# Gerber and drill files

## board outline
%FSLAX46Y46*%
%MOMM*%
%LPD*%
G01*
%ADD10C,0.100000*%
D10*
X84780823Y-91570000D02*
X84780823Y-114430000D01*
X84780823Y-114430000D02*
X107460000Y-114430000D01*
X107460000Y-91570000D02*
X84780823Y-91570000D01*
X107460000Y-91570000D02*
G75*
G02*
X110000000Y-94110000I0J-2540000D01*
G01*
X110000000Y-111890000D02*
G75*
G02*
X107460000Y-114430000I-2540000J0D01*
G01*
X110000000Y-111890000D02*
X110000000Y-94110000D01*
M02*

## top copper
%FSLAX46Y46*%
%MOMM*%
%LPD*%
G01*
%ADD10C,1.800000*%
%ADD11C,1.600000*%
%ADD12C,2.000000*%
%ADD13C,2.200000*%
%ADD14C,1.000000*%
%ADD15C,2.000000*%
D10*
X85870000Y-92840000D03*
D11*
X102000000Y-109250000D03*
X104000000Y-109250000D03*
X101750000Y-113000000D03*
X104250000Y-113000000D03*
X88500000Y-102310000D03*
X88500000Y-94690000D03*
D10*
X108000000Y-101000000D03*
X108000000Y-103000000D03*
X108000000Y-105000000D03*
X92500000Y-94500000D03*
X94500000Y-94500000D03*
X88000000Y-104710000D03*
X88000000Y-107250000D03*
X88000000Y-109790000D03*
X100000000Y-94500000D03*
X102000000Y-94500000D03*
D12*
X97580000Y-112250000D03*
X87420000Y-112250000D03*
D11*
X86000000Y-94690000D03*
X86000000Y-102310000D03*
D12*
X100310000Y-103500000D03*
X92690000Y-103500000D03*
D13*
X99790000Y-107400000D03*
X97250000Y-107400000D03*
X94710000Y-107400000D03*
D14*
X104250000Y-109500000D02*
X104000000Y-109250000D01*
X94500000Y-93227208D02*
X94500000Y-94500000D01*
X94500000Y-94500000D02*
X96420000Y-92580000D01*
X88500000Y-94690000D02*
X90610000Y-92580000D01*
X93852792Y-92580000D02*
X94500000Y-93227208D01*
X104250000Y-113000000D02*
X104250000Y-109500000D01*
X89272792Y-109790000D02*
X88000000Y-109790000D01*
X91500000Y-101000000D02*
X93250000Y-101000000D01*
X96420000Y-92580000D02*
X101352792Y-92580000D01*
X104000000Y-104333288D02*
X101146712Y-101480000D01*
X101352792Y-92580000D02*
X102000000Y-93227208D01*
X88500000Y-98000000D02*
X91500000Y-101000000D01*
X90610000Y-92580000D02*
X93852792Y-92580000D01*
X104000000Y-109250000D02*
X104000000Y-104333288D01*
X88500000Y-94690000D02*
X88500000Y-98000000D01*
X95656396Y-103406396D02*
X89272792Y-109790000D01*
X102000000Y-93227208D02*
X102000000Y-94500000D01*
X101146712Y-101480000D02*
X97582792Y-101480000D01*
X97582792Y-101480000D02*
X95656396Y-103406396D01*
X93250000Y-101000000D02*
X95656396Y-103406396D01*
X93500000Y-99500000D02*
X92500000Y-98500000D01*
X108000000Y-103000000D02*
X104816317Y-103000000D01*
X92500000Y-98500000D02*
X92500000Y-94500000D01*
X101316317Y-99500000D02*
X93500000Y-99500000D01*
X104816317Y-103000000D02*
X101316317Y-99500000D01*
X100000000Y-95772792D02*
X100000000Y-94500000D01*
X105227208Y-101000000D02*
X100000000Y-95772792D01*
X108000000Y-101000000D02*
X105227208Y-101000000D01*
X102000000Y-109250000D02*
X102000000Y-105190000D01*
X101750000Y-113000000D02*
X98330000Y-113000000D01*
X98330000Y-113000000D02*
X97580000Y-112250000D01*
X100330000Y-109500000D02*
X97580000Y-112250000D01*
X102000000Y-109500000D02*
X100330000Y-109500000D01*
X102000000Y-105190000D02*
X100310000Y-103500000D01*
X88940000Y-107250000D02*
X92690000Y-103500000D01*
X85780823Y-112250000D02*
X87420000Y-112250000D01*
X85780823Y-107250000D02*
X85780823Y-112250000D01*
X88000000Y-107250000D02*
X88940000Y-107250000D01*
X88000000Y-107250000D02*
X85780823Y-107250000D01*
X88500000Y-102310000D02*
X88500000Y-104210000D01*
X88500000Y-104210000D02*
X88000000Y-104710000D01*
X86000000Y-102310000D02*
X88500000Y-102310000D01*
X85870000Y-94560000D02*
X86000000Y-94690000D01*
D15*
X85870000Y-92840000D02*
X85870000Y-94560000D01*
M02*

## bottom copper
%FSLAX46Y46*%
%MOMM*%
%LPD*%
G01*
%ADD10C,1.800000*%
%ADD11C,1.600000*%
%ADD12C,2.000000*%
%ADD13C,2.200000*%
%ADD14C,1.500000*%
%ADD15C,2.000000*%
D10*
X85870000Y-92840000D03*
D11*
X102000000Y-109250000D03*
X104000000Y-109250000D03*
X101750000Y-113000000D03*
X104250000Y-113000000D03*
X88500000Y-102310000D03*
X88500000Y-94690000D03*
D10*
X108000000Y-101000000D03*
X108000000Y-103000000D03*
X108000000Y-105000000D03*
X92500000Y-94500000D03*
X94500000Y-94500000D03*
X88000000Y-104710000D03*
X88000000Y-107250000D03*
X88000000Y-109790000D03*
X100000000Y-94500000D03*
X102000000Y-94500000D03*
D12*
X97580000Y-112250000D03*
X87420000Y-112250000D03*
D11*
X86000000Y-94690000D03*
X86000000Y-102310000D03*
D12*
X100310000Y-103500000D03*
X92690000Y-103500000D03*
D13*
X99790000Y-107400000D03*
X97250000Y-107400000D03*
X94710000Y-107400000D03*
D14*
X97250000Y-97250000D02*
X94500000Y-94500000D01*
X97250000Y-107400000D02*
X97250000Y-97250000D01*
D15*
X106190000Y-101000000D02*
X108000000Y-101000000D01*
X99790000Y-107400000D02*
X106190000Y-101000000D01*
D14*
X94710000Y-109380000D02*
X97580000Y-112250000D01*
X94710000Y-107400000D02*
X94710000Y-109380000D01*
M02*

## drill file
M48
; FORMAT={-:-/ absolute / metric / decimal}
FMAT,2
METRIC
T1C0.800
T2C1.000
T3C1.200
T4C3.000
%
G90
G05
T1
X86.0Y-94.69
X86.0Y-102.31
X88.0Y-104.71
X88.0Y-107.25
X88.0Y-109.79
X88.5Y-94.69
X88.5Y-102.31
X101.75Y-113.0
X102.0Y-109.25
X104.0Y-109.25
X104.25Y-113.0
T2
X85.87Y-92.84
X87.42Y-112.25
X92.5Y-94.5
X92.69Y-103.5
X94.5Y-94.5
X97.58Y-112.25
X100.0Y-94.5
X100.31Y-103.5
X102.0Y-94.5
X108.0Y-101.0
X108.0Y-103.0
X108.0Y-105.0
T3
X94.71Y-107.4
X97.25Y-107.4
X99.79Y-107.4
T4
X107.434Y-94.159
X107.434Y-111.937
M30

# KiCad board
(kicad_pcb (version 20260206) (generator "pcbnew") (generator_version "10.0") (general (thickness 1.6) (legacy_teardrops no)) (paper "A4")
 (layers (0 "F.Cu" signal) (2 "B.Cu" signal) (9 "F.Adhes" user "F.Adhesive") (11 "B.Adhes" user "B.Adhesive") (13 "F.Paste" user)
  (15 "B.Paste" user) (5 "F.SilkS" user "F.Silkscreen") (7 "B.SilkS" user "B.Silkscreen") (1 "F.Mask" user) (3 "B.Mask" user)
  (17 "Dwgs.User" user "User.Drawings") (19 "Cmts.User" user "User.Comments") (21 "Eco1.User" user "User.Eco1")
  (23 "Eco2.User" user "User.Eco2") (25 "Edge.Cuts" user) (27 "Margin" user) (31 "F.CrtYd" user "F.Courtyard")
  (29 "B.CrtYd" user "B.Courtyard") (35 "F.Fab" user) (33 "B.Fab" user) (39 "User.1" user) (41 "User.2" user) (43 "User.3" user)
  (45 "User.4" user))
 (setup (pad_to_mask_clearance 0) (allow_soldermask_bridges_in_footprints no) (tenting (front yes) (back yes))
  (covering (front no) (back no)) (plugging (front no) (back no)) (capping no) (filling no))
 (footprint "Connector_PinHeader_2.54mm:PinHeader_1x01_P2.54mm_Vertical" (layer "F.Cu") (at 85.87 92.84)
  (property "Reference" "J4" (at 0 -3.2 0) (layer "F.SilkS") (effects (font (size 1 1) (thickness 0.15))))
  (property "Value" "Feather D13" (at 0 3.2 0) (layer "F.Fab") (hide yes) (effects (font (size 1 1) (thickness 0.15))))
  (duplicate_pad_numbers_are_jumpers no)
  (pad "1" thru_hole circle (at 0 0) (size 1.8 1.8) (drill 1) (layers "*.Cu" "*.Mask") (remove_unused_layers no) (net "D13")))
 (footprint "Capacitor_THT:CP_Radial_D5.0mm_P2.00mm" (layer "F.Cu") (at 103 109.25)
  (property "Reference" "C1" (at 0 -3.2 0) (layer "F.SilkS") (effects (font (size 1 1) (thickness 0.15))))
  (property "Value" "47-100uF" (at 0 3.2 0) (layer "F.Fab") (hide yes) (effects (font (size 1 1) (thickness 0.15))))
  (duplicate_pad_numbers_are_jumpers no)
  (pad "1" thru_hole circle (at -1 0) (size 1.6 1.6) (drill 0.8) (layers "*.Cu" "*.Mask") (remove_unused_layers no) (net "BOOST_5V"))
  (pad "2" thru_hole circle (at 1 0) (size 1.6 1.6) (drill 0.8) (layers "*.Cu" "*.Mask") (remove_unused_layers no) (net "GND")))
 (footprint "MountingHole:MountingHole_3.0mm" (layer "F.Cu") (at 107.434 111.937)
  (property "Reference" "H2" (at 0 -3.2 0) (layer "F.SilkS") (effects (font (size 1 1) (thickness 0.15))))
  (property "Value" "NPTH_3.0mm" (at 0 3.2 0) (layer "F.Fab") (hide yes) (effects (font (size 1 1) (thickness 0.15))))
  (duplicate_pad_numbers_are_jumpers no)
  (pad "" np_thru_hole circle (at 0 0) (size 3 3) (drill 3) (layers "*.Cu" "*.Mask")))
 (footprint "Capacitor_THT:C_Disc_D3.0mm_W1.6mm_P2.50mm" (layer "F.Cu") (at 103 113)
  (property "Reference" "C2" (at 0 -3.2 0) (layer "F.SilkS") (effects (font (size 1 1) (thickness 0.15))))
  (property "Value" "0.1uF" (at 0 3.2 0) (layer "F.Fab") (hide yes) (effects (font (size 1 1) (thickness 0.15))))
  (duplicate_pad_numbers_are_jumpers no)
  (pad "1" thru_hole circle (at -1.25 0) (size 1.6 1.6) (drill 0.8) (layers "*.Cu" "*.Mask") (remove_unused_layers no) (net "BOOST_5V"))
  (pad "2" thru_hole circle (at 1.25 0) (size 1.6 1.6) (drill 0.8) (layers "*.Cu" "*.Mask") (remove_unused_layers no) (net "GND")))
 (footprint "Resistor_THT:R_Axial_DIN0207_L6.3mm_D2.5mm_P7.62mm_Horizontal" (layer "F.Cu") (at 88.5 98.5 90)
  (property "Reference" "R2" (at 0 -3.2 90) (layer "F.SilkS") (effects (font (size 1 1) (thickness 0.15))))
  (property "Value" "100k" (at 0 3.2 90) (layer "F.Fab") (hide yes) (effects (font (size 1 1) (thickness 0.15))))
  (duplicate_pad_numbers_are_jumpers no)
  (pad "1" thru_hole circle (at -3.81 0 90) (size 1.6 1.6) (drill 0.8) (layers "*.Cu" "*.Mask") (remove_unused_layers no)
   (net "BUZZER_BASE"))
  (pad "2" thru_hole circle (at 3.81 0 90) (size 1.6 1.6) (drill 0.8) (layers "*.Cu" "*.Mask") (remove_unused_layers no) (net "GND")))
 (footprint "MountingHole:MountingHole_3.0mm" (layer "F.Cu") (at 107.434 94.1586)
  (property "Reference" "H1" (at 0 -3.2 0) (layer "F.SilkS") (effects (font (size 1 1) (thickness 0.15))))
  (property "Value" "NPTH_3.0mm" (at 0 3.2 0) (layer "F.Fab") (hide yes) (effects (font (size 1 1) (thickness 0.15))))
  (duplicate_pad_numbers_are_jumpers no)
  (pad "" np_thru_hole circle (at 0 0) (size 3 3) (drill 3) (layers "*.Cu" "*.Mask")))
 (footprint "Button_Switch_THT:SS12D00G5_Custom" (layer "F.Cu") (at 108 103 -90)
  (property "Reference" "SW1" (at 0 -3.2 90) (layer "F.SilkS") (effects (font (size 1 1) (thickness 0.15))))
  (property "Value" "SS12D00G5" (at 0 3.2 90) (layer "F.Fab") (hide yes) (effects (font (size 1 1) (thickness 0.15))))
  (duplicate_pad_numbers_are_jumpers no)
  (pad "1" thru_hole circle (at -2 0 270) (size 1.8 1.8) (drill 1) (layers "*.Cu" "*.Mask") (remove_unused_layers no) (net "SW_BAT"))
  (pad "2" thru_hole circle (at 0 0 270) (size 1.8 1.8) (drill 1) (layers "*.Cu" "*.Mask") (remove_unused_layers no) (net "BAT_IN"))
  (pad "3" thru_hole circle (at 2 0 270) (size 1.8 1.8) (drill 1) (layers "*.Cu" "*.Mask") (remove_unused_layers no)))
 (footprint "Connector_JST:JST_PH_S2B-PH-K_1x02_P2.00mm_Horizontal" (layer "F.Cu") (at 93.5 94.5)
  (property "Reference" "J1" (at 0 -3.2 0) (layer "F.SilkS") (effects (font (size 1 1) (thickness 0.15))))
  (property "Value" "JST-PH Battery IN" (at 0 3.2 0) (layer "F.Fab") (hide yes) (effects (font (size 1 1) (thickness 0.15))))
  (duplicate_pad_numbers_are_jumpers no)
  (pad "1" thru_hole circle (at -1 0) (size 1.8 1.8) (drill 1) (layers "*.Cu" "*.Mask") (remove_unused_layers no) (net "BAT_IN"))
  (pad "2" thru_hole circle (at 1 0) (size 1.8 1.8) (drill 1) (layers "*.Cu" "*.Mask") (remove_unused_layers no) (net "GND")))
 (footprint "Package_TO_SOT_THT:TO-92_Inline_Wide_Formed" (layer "F.Cu") (at 88 107.25 -90)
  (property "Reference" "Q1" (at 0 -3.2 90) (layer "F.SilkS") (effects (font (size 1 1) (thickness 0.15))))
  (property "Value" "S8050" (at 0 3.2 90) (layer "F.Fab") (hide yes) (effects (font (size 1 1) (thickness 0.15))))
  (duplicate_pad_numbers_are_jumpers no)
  (pad "1" thru_hole circle (at -2.54 0 270) (size 1.8 1.8) (drill 0.8) (layers "*.Cu" "*.Mask") (remove_unused_layers no)
   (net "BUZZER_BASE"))
  (pad "2" thru_hole circle (at 0 0 270) (size 1.8 1.8) (drill 0.8) (layers "*.Cu" "*.Mask") (remove_unused_layers no) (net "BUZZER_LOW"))
  (pad "3" thru_hole circle (at 2.54 0 270) (size 1.8 1.8) (drill 0.8) (layers "*.Cu" "*.Mask") (remove_unused_layers no) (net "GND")))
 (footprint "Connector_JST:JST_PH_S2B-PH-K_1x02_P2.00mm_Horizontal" (layer "F.Cu") (at 101 94.5)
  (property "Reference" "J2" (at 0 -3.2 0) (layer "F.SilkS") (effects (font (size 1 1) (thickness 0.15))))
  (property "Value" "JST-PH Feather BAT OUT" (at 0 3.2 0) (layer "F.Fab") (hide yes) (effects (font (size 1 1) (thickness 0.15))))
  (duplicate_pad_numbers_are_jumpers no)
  (pad "1" thru_hole circle (at -1 0) (size 1.8 1.8) (drill 1) (layers "*.Cu" "*.Mask") (remove_unused_layers no) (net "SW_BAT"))
  (pad "2" thru_hole circle (at 1 0) (size 1.8 1.8) (drill 1) (layers "*.Cu" "*.Mask") (remove_unused_layers no) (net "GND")))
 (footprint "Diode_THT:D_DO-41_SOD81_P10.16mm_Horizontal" (layer "F.Cu") (at 92.5 112.25 180)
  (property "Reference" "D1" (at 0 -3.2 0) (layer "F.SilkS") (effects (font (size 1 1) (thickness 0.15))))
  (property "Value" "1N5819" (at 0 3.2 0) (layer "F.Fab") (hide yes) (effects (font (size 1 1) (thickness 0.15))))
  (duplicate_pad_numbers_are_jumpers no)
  (pad "1" thru_hole circle (at -5.08 0 180) (size 2 2) (drill 1) (layers "*.Cu" "*.Mask") (remove_unused_layers no) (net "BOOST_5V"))
  (pad "2" thru_hole circle (at 5.08 0 180) (size 2 2) (drill 1) (layers "*.Cu" "*.Mask") (remove_unused_layers no) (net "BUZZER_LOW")))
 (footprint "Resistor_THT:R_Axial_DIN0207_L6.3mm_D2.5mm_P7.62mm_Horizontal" (layer "F.Cu") (at 86 98.5 -90)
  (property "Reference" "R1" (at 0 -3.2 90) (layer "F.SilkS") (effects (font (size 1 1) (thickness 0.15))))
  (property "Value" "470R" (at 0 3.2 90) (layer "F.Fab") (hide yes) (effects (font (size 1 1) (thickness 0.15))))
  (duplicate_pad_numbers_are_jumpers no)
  (pad "1" thru_hole circle (at -3.81 0 270) (size 1.6 1.6) (drill 0.8) (layers "*.Cu" "*.Mask") (remove_unused_layers no) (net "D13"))
  (pad "2" thru_hole circle (at 3.81 0 270) (size 1.6 1.6) (drill 0.8) (layers "*.Cu" "*.Mask") (remove_unused_layers no)
   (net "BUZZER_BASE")))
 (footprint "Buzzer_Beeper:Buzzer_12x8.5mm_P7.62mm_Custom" (layer "F.Cu") (at 96.5 103.5 180)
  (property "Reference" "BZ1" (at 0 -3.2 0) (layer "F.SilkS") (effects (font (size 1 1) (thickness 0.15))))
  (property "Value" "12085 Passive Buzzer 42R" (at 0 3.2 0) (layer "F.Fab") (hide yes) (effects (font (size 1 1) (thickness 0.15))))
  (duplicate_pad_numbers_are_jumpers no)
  (pad "1" thru_hole circle (at -3.81 0 180) (size 2 2) (drill 1) (layers "*.Cu" "*.Mask") (remove_unused_layers no) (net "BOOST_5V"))
  (pad "2" thru_hole circle (at 3.81 0 180) (size 2 2) (drill 1) (layers "*.Cu" "*.Mask") (remove_unused_layers no) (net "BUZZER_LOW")))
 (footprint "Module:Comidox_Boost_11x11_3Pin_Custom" (layer "B.Cu") (at 97.25 103.25 90)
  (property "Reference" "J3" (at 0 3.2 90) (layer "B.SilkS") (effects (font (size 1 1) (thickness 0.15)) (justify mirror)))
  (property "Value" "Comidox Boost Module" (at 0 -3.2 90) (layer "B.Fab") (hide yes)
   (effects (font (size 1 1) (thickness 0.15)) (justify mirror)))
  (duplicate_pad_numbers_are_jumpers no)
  (pad "1" thru_hole circle (at -4.15 2.54 90) (size 2.2 2.2) (drill 1.2) (layers "*.Cu" "*.Mask") (remove_unused_layers no) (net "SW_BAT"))
  (pad "2" thru_hole circle (at -4.15 0 90) (size 2.2 2.2) (drill 1.2) (layers "*.Cu" "*.Mask") (remove_unused_layers no) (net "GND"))
  (pad "3" thru_hole circle (at -4.15 -2.54 90) (size 2.2 2.2) (drill 1.2) (layers "*.Cu" "*.Mask") (remove_unused_layers no)
   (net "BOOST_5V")))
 (gr_line (start 84.780823 91.57) (end 84.780823 114.43) (stroke (width 0.1) (type default)) (layer "Edge.Cuts"))
 (gr_line (start 84.780823 114.43) (end 107.46 114.43) (stroke (width 0.1) (type default)) (layer "Edge.Cuts"))
 (gr_line (start 107.46 91.57) (end 84.780823 91.57) (stroke (width 0.1) (type default)) (layer "Edge.Cuts"))
 (gr_arc (start 107.46 91.57) (mid 109.256051 92.313949) (end 110 94.11) (stroke (width 0.1) (type default)) (layer "Edge.Cuts"))
 (gr_arc (start 110 111.89) (mid 109.256051 113.686051) (end 107.46 114.43) (stroke (width 0.1) (type default)) (layer "Edge.Cuts"))
 (gr_line (start 110 111.89) (end 110 94.11) (stroke (width 0.1) (type default)) (layer "Edge.Cuts"))
 (segment (start 104.25 109.5) (end 104 109.25) (width 1) (layer "F.Cu") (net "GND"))
 (segment (start 94.5 93.227208) (end 94.5 94.5) (width 1) (layer "F.Cu") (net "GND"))
 (segment (start 94.5 94.5) (end 96.42 92.58) (width 1) (layer "F.Cu") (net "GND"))
 (segment (start 88.5 94.69) (end 90.61 92.58) (width 1) (layer "F.Cu") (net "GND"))
 (segment (start 93.852792 92.58) (end 94.5 93.227208) (width 1) (layer "F.Cu") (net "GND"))
 (segment (start 104.25 113) (end 104.25 109.5) (width 1) (layer "F.Cu") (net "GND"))
 (segment (start 89.272792 109.79) (end 88 109.79) (width 1) (layer "F.Cu") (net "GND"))
 (segment (start 91.5 101) (end 93.25 101) (width 1) (layer "F.Cu") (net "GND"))
 (segment (start 96.42 92.58) (end 101.352792 92.58) (width 1) (layer "F.Cu") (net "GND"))
 (segment (start 104 104.333288) (end 101.146712 101.48) (width 1) (layer "F.Cu") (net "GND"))
 (segment (start 101.352792 92.58) (end 102 93.227208) (width 1) (layer "F.Cu") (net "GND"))
 (segment (start 88.5 98) (end 91.5 101) (width 1) (layer "F.Cu") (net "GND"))
 (segment (start 90.61 92.58) (end 93.852792 92.58) (width 1) (layer "F.Cu") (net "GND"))
 (segment (start 104 109.25) (end 104 104.333288) (width 1) (layer "F.Cu") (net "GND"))
 (segment (start 88.5 94.69) (end 88.5 98) (width 1) (layer "F.Cu") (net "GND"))
 (segment (start 95.656396 103.406396) (end 89.272792 109.79) (width 1) (layer "F.Cu") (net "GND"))
 (segment (start 102 93.227208) (end 102 94.5) (width 1) (layer "F.Cu") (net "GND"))
 (segment (start 101.146712 101.48) (end 97.582792 101.48) (width 1) (layer "F.Cu") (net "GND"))
 (segment (start 97.582792 101.48) (end 95.656396 103.406396) (width 1) (layer "F.Cu") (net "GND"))
 (segment (start 93.25 101) (end 95.656396 103.406396) (width 1) (layer "F.Cu") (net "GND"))
 (segment (start 97.25 97.25) (end 94.5 94.5) (width 1.5) (layer "B.Cu") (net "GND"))
 (segment (start 97.25 107.4) (end 97.25 97.25) (width 1.5) (layer "B.Cu") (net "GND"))
 (segment (start 93.5 99.5) (end 92.5 98.5) (width 1) (layer "F.Cu") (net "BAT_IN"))
 (segment (start 108 103) (end 104.816317 103) (width 1) (layer "F.Cu") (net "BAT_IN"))
 (segment (start 92.5 98.5) (end 92.5 94.5) (width 1) (layer "F.Cu") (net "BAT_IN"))
 (segment (start 101.316317 99.5) (end 93.5 99.5) (width 1) (layer "F.Cu") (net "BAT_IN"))
 (segment (start 104.816317 103) (end 101.316317 99.5) (width 1) (layer "F.Cu") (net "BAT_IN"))
 (segment (start 100 95.772792) (end 100 94.5) (width 1) (layer "F.Cu") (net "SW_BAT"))
 (segment (start 105.227208 101) (end 100 95.772792) (width 1) (layer "F.Cu") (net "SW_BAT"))
 (segment (start 108 101) (end 105.227208 101) (width 1) (layer "F.Cu") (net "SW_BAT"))
 (segment (start 106.19 101) (end 108 101) (width 2) (layer "B.Cu") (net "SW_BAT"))
 (segment (start 99.79 107.4) (end 106.19 101) (width 2) (layer "B.Cu") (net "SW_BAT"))
 (segment (start 102 109.25) (end 102 105.19) (width 1) (layer "F.Cu") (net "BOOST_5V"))
 (segment (start 101.75 113) (end 98.33 113) (width 1) (layer "F.Cu") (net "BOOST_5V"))
 (segment (start 98.33 113) (end 97.58 112.25) (width 1) (layer "F.Cu") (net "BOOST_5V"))
 (segment (start 100.33 109.5) (end 97.58 112.25) (width 1) (layer "F.Cu") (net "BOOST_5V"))
 (segment (start 102 109.5) (end 100.33 109.5) (width 1) (layer "F.Cu") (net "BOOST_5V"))
 (segment (start 102 105.19) (end 100.31 103.5) (width 1) (layer "F.Cu") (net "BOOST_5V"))
 (segment (start 94.71 109.38) (end 97.58 112.25) (width 1.5) (layer "B.Cu") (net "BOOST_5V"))
 (segment (start 94.71 107.4) (end 94.71 109.38) (width 1.5) (layer "B.Cu") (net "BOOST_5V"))
 (segment (start 88.94 107.25) (end 92.69 103.5) (width 1) (layer "F.Cu") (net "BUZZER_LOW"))
 (segment (start 85.780823 112.25) (end 87.42 112.25) (width 1) (layer "F.Cu") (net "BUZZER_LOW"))
 (segment (start 85.780823 107.25) (end 85.780823 112.25) (width 1) (layer "F.Cu") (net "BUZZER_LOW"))
 (segment (start 88 107.25) (end 88.94 107.25) (width 1) (layer "F.Cu") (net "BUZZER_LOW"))
 (segment (start 88 107.25) (end 85.780823 107.25) (width 1) (layer "F.Cu") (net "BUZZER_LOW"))
 (segment (start 88.5 102.31) (end 88.5 104.21) (width 1) (layer "F.Cu") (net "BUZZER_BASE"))
 (segment (start 88.5 104.21) (end 88 104.71) (width 1) (layer "F.Cu") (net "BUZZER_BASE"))
 (segment (start 86 102.31) (end 88.5 102.31) (width 1) (layer "F.Cu") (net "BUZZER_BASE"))
 (segment (start 85.87 94.56) (end 86 94.69) (width 1) (layer "F.Cu") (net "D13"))
 (segment (start 85.87 92.84) (end 85.87 94.56) (width 2) (layer "F.Cu") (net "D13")))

